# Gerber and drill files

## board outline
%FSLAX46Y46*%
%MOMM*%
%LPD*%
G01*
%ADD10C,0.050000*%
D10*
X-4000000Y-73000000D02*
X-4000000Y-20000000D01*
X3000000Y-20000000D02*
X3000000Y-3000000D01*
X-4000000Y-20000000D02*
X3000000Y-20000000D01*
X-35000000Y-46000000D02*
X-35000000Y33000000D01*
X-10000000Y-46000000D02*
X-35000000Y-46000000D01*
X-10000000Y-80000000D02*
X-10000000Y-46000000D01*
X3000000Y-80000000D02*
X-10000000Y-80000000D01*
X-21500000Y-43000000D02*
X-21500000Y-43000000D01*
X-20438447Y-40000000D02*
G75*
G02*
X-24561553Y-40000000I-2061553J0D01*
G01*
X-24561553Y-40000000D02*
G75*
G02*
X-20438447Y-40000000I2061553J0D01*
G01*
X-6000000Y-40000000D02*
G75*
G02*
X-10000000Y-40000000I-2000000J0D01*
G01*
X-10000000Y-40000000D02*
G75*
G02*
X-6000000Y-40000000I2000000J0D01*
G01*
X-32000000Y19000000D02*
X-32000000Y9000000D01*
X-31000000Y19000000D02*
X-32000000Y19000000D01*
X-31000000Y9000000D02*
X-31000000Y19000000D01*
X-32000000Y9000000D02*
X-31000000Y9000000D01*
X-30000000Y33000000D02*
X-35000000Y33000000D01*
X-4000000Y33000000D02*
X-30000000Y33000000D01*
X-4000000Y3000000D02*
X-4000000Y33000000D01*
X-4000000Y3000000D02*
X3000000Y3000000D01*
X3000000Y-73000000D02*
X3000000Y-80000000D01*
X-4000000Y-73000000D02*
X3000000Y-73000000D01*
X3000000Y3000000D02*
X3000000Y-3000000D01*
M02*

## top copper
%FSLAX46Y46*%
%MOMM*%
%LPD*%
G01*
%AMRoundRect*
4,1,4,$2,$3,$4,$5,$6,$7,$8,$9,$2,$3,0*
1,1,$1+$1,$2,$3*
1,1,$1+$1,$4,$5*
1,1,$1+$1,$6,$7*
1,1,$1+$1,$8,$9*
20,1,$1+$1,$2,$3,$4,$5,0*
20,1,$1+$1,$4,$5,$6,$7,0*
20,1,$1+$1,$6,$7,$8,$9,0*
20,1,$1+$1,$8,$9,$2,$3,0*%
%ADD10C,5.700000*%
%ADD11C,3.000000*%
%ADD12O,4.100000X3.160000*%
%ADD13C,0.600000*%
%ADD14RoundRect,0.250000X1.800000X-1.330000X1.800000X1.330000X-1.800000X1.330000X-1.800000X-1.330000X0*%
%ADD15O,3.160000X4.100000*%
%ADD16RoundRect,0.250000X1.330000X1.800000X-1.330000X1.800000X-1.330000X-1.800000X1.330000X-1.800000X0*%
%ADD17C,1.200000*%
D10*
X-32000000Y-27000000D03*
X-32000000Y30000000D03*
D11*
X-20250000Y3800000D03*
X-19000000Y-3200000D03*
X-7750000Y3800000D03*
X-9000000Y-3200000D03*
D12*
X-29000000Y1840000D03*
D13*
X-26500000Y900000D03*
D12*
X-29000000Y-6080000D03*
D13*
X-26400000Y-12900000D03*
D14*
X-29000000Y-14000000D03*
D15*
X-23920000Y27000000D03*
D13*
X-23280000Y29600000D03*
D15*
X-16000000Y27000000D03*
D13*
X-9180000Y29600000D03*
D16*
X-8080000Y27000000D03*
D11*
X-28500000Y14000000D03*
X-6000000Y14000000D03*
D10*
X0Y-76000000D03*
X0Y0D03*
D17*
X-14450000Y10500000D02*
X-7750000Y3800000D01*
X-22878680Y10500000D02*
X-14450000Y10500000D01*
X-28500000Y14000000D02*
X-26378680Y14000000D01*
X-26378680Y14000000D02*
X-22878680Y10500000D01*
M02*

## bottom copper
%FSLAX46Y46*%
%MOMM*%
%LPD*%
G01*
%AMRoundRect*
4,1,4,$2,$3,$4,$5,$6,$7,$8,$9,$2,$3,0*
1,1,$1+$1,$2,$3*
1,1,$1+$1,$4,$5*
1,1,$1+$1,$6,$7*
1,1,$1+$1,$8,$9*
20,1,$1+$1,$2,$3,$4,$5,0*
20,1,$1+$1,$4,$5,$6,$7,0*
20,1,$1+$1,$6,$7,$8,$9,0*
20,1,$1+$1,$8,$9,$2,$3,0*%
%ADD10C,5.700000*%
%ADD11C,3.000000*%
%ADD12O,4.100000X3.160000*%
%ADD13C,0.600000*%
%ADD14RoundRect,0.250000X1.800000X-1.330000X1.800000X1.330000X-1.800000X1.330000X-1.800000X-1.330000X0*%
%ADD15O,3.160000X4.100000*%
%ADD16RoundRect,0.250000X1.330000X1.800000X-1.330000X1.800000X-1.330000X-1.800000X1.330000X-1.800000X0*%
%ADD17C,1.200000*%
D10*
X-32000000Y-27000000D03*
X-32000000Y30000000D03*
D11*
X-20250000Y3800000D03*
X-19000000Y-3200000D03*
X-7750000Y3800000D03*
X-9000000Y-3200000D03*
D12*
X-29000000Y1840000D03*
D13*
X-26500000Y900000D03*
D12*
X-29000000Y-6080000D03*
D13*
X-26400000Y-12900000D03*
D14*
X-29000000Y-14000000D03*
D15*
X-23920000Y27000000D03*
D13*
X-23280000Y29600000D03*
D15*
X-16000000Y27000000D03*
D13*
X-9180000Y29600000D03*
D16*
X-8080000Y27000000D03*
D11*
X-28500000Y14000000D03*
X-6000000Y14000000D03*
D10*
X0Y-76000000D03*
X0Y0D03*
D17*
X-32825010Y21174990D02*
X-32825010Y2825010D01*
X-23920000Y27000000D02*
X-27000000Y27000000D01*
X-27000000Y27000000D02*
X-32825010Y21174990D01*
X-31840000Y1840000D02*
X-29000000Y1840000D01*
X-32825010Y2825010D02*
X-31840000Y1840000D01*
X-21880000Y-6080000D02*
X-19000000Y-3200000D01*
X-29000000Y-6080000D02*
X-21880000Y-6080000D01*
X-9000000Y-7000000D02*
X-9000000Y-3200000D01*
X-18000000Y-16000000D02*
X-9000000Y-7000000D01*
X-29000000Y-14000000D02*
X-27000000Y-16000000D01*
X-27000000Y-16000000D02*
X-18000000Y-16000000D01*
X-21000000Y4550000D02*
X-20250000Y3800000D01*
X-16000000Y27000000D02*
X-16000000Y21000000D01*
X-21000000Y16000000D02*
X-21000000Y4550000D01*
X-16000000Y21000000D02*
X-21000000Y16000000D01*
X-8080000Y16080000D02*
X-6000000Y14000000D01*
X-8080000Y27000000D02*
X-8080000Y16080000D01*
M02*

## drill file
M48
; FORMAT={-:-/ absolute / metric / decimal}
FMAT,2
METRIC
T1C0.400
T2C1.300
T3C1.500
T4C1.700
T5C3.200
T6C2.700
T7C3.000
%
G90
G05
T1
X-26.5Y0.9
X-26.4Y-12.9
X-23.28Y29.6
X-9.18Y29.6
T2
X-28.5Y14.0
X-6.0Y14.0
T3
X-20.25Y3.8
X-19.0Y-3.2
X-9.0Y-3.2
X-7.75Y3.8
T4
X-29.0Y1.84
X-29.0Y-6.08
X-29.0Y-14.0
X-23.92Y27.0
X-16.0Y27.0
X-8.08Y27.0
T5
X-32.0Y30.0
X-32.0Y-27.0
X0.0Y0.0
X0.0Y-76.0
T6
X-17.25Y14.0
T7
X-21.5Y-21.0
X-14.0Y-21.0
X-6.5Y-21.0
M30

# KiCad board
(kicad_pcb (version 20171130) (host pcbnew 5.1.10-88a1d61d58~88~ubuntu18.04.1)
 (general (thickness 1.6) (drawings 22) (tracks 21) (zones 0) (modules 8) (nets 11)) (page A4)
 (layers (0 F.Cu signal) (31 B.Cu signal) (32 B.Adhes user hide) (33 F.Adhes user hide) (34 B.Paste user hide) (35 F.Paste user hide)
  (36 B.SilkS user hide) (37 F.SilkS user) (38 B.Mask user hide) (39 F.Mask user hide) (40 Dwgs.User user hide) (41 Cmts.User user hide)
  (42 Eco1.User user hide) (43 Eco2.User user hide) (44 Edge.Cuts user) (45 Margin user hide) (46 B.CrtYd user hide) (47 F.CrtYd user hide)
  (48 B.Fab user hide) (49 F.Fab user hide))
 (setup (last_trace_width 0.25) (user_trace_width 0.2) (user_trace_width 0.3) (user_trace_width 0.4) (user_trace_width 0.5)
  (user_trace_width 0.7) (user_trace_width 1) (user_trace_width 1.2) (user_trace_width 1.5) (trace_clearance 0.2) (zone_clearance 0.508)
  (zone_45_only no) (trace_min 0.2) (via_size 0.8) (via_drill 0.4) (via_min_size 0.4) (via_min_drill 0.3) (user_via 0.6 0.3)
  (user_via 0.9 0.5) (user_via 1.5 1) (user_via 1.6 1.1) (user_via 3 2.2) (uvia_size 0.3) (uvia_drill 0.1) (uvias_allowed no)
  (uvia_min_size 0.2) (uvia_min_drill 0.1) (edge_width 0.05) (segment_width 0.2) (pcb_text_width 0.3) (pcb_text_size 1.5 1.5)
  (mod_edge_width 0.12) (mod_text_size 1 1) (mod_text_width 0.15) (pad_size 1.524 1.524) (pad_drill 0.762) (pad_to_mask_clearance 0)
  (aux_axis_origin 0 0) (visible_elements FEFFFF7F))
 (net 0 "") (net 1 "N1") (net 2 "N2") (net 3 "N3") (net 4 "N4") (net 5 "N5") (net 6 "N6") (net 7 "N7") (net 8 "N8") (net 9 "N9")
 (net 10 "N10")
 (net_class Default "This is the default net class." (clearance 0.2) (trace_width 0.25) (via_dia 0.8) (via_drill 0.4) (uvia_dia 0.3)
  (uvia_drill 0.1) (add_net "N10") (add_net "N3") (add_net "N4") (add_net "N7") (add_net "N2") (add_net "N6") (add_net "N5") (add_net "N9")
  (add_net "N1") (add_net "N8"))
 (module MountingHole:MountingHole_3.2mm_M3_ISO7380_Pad (layer F.Cu) (at -32 27)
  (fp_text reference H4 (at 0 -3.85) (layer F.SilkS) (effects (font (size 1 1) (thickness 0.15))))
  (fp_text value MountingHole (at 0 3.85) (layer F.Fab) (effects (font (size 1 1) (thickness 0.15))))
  (pad 1 thru_hole circle (at 0 0) (size 5.7 5.7) (drill 3.2) (layers *.Cu *.Mask)))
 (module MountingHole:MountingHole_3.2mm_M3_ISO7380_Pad (layer F.Cu) (at -32 -30)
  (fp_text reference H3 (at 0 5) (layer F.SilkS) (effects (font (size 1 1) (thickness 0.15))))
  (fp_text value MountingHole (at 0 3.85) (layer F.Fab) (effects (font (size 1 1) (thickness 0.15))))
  (pad 1 thru_hole circle (at 0 0) (size 5.7 5.7) (drill 3.2) (layers *.Cu *.Mask)))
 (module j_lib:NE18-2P (layer F.Cu) (at -14 21 270)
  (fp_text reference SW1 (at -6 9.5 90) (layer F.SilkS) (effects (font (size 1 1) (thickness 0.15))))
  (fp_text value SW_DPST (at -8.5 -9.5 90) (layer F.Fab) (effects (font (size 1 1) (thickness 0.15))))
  (pad "" np_thru_hole circle (at 0 7.5 270) (size 3 3) (drill 3) (layers *.Cu *.Mask))
  (pad "" np_thru_hole circle (at 0 0 270) (size 3 3) (drill 3) (layers *.Cu *.Mask))
  (pad "" np_thru_hole circle (at 0 -7.5 270) (size 3 3) (drill 3) (layers *.Cu *.Mask))
  (pad 4 thru_hole circle (at -24.8 6.25 270) (size 3 3) (drill 1.5) (layers *.Cu *.Mask) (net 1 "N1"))
  (pad 3 thru_hole circle (at -17.8 5 270) (size 3 3) (drill 1.5) (layers *.Cu *.Mask) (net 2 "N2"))
  (pad 2 thru_hole circle (at -24.8 -6.25 270) (size 3 3) (drill 1.5) (layers *.Cu *.Mask) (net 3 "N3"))
  (pad 1 thru_hole circle (at -17.8 -5 270) (size 3 3) (drill 1.5) (layers *.Cu *.Mask) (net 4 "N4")))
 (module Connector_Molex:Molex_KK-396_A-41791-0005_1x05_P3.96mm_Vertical (layer F.Cu) (at -29 14 90)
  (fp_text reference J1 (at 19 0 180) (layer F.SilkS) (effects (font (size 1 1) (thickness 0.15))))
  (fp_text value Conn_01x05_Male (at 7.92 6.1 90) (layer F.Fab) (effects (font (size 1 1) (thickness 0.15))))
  (pad 5 thru_hole oval (at 15.84 0 90) (size 3.16 4.1) (drill 1.7) (layers *.Cu *.Mask) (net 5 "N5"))
  (pad 4 thru_hole circle (at 14.9 2.5 90) (size 0.6 0.6) (drill 0.4) (layers *.Cu *.Mask) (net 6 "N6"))
  (pad 3 thru_hole oval (at 7.92 0 90) (size 3.16 4.1) (drill 1.7) (layers *.Cu *.Mask) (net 2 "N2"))
  (pad 2 thru_hole circle (at 1.1 2.6 90) (size 0.6 0.6) (drill 0.4) (layers *.Cu *.Mask) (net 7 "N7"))
  (pad 1 thru_hole roundrect (at 0 0 90) (size 3.16 4.1) (drill 1.7) (layers *.Cu *.Mask) (roundrect_rratio 0.07911392405063292)
   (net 4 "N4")))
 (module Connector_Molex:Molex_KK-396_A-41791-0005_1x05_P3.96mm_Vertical (layer F.Cu) (at -8.08 -27 180)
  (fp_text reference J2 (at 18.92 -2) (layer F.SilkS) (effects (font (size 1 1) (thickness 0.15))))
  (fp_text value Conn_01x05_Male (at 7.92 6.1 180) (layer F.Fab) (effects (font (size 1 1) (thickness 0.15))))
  (pad 5 thru_hole oval (at 15.84 0 180) (size 3.16 4.1) (drill 1.7) (layers *.Cu *.Mask) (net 5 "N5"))
  (pad 4 thru_hole circle (at 15.2 2.6 180) (size 0.6 0.6) (drill 0.4) (layers *.Cu *.Mask) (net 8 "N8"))
  (pad 3 thru_hole oval (at 7.92 0 180) (size 3.16 4.1) (drill 1.7) (layers *.Cu *.Mask) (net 1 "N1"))
  (pad 2 thru_hole circle (at 1.1 2.6 180) (size 0.6 0.6) (drill 0.4) (layers *.Cu *.Mask) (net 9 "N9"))
  (pad 1 thru_hole roundrect (at 0 0 180) (size 3.16 4.1) (drill 1.7) (layers *.Cu *.Mask) (roundrect_rratio 0.07911392405063292)
   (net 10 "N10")))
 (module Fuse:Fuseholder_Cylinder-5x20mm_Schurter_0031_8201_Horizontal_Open (layer F.Cu) (at -6 -14 180)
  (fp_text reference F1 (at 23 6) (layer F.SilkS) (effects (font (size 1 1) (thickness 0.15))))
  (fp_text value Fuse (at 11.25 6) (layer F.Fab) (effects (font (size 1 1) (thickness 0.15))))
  (pad "" np_thru_hole circle (at 11.25 0 180) (size 2.7 2.7) (drill 2.7) (layers *.Cu *.Mask))
  (pad 2 thru_hole circle (at 22.5 0 180) (size 3 3) (drill 1.3) (layers *.Cu *.Mask) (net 3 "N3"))
  (pad 1 thru_hole circle (at 0 0 180) (size 3 3) (drill 1.3) (layers *.Cu *.Mask) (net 10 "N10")))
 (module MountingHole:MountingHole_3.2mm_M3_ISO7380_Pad (layer F.Cu) (at 0 76)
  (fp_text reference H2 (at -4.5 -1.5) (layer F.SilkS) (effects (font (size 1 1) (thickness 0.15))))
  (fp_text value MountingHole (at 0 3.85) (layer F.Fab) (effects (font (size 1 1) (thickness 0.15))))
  (pad 1 thru_hole circle (at 0 0) (size 5.7 5.7) (drill 3.2) (layers *.Cu *.Mask)))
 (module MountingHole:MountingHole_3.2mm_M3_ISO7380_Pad (layer F.Cu) (at 0 0)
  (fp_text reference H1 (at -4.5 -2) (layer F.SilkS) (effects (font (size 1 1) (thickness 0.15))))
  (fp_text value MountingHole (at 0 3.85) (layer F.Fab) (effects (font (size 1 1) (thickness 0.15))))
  (pad 1 thru_hole circle (at 0 0) (size 5.7 5.7) (drill 3.2) (layers *.Cu *.Mask)))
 (gr_line (start -4 73) (end -4 20) (layer Edge.Cuts) (width 0.05))
 (gr_line (start 3 20) (end 3 3) (layer Edge.Cuts) (width 0.05))
 (gr_line (start -4 20) (end 3 20) (layer Edge.Cuts) (width 0.05))
 (gr_line (start -35 46) (end -35 -33) (layer Edge.Cuts) (width 0.05))
 (gr_line (start -10 46) (end -35 46) (layer Edge.Cuts) (width 0.05))
 (gr_line (start -10 80) (end -10 46) (layer Edge.Cuts) (width 0.05))
 (gr_line (start 3 80) (end -10 80) (layer Edge.Cuts) (width 0.05))
 (gr_line (start -21.5 43) (end -21.5 43) (layer Edge.Cuts) (width 0.05))
 (gr_circle (center -22.5 40) (end -23 42) (layer Edge.Cuts) (width 0.05))
 (gr_circle (center -8 40) (end -6 40) (layer Edge.Cuts) (width 0.05))
 (gr_line (start -32 -19) (end -32 -9) (layer Edge.Cuts) (width 0.05))
 (gr_line (start -31 -19) (end -32 -19) (layer Edge.Cuts) (width 0.05))
 (gr_line (start -31 -9) (end -31 -19) (layer Edge.Cuts) (width 0.05))
 (gr_line (start -32 -9) (end -31 -9) (layer Edge.Cuts) (width 0.05))
 (gr_line (start -30 -33) (end -35 -33) (layer Edge.Cuts) (width 0.05))
 (gr_line (start -4 -33) (end -30 -33) (layer Edge.Cuts) (width 0.05))
 (gr_line (start -4 -3) (end -4 -33) (layer Edge.Cuts) (width 0.05))
 (gr_line (start -4 -3) (end 3 -3) (layer Edge.Cuts) (width 0.05))
 (gr_line (start 3 73) (end 3 80) (layer Edge.Cuts) (width 0.05))
 (gr_line (start -4 73) (end 3 73) (layer Edge.Cuts) (width 0.05))
 (gr_line (start 3 -3) (end 3 3) (layer Edge.Cuts) (width 0.05))
 (segment (start -32.82501 -21.17499) (end -32.82501 -2.82501) (width 1.2) (layer B.Cu) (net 5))
 (segment (start -23.92 -27) (end -27 -27) (width 1.2) (layer B.Cu) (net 5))
 (segment (start -27 -27) (end -32.82501 -21.17499) (width 1.2) (layer B.Cu) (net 5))
 (segment (start -31.84 -1.84) (end -29 -1.84) (width 1.2) (layer B.Cu) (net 5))
 (segment (start -32.82501 -2.82501) (end -31.84 -1.84) (width 1.2) (layer B.Cu) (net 5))
 (segment (start -21.88 6.08) (end -19 3.2) (width 1.2) (layer B.Cu) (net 2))
 (segment (start -29 6.08) (end -21.88 6.08) (width 1.2) (layer B.Cu) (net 2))
 (segment (start -9 7) (end -9 3.2) (width 1.2) (layer B.Cu) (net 4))
 (segment (start -18 16) (end -9 7) (width 1.2) (layer B.Cu) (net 4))
 (segment (start -29 14) (end -27 16) (width 1.2) (layer B.Cu) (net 4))
 (segment (start -27 16) (end -18 16) (width 1.2) (layer B.Cu) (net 4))
 (segment (start -21 -4.55) (end -20.25 -3.8) (width 1.2) (layer B.Cu) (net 1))
 (segment (start -16 -27) (end -16 -21) (width 1.2) (layer B.Cu) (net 1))
 (segment (start -21 -16) (end -21 -4.55) (width 1.2) (layer B.Cu) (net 1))
 (segment (start -16 -21) (end -21 -16) (width 1.2) (layer B.Cu) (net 1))
 (segment (start -14.45 -10.5) (end -7.75 -3.8) (width 1.2) (layer F.Cu) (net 3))
 (segment (start -22.87868 -10.5) (end -14.45 -10.5) (width 1.2) (layer F.Cu) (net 3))
 (segment (start -28.5 -14) (end -26.37868 -14) (width 1.2) (layer F.Cu) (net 3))
 (segment (start -26.37868 -14) (end -22.87868 -10.5) (width 1.2) (layer F.Cu) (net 3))
 (segment (start -8.08 -16.08) (end -6 -14) (width 1.2) (layer B.Cu) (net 10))
 (segment (start -8.08 -27) (end -8.08 -16.08) (width 1.2) (layer B.Cu) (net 10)))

